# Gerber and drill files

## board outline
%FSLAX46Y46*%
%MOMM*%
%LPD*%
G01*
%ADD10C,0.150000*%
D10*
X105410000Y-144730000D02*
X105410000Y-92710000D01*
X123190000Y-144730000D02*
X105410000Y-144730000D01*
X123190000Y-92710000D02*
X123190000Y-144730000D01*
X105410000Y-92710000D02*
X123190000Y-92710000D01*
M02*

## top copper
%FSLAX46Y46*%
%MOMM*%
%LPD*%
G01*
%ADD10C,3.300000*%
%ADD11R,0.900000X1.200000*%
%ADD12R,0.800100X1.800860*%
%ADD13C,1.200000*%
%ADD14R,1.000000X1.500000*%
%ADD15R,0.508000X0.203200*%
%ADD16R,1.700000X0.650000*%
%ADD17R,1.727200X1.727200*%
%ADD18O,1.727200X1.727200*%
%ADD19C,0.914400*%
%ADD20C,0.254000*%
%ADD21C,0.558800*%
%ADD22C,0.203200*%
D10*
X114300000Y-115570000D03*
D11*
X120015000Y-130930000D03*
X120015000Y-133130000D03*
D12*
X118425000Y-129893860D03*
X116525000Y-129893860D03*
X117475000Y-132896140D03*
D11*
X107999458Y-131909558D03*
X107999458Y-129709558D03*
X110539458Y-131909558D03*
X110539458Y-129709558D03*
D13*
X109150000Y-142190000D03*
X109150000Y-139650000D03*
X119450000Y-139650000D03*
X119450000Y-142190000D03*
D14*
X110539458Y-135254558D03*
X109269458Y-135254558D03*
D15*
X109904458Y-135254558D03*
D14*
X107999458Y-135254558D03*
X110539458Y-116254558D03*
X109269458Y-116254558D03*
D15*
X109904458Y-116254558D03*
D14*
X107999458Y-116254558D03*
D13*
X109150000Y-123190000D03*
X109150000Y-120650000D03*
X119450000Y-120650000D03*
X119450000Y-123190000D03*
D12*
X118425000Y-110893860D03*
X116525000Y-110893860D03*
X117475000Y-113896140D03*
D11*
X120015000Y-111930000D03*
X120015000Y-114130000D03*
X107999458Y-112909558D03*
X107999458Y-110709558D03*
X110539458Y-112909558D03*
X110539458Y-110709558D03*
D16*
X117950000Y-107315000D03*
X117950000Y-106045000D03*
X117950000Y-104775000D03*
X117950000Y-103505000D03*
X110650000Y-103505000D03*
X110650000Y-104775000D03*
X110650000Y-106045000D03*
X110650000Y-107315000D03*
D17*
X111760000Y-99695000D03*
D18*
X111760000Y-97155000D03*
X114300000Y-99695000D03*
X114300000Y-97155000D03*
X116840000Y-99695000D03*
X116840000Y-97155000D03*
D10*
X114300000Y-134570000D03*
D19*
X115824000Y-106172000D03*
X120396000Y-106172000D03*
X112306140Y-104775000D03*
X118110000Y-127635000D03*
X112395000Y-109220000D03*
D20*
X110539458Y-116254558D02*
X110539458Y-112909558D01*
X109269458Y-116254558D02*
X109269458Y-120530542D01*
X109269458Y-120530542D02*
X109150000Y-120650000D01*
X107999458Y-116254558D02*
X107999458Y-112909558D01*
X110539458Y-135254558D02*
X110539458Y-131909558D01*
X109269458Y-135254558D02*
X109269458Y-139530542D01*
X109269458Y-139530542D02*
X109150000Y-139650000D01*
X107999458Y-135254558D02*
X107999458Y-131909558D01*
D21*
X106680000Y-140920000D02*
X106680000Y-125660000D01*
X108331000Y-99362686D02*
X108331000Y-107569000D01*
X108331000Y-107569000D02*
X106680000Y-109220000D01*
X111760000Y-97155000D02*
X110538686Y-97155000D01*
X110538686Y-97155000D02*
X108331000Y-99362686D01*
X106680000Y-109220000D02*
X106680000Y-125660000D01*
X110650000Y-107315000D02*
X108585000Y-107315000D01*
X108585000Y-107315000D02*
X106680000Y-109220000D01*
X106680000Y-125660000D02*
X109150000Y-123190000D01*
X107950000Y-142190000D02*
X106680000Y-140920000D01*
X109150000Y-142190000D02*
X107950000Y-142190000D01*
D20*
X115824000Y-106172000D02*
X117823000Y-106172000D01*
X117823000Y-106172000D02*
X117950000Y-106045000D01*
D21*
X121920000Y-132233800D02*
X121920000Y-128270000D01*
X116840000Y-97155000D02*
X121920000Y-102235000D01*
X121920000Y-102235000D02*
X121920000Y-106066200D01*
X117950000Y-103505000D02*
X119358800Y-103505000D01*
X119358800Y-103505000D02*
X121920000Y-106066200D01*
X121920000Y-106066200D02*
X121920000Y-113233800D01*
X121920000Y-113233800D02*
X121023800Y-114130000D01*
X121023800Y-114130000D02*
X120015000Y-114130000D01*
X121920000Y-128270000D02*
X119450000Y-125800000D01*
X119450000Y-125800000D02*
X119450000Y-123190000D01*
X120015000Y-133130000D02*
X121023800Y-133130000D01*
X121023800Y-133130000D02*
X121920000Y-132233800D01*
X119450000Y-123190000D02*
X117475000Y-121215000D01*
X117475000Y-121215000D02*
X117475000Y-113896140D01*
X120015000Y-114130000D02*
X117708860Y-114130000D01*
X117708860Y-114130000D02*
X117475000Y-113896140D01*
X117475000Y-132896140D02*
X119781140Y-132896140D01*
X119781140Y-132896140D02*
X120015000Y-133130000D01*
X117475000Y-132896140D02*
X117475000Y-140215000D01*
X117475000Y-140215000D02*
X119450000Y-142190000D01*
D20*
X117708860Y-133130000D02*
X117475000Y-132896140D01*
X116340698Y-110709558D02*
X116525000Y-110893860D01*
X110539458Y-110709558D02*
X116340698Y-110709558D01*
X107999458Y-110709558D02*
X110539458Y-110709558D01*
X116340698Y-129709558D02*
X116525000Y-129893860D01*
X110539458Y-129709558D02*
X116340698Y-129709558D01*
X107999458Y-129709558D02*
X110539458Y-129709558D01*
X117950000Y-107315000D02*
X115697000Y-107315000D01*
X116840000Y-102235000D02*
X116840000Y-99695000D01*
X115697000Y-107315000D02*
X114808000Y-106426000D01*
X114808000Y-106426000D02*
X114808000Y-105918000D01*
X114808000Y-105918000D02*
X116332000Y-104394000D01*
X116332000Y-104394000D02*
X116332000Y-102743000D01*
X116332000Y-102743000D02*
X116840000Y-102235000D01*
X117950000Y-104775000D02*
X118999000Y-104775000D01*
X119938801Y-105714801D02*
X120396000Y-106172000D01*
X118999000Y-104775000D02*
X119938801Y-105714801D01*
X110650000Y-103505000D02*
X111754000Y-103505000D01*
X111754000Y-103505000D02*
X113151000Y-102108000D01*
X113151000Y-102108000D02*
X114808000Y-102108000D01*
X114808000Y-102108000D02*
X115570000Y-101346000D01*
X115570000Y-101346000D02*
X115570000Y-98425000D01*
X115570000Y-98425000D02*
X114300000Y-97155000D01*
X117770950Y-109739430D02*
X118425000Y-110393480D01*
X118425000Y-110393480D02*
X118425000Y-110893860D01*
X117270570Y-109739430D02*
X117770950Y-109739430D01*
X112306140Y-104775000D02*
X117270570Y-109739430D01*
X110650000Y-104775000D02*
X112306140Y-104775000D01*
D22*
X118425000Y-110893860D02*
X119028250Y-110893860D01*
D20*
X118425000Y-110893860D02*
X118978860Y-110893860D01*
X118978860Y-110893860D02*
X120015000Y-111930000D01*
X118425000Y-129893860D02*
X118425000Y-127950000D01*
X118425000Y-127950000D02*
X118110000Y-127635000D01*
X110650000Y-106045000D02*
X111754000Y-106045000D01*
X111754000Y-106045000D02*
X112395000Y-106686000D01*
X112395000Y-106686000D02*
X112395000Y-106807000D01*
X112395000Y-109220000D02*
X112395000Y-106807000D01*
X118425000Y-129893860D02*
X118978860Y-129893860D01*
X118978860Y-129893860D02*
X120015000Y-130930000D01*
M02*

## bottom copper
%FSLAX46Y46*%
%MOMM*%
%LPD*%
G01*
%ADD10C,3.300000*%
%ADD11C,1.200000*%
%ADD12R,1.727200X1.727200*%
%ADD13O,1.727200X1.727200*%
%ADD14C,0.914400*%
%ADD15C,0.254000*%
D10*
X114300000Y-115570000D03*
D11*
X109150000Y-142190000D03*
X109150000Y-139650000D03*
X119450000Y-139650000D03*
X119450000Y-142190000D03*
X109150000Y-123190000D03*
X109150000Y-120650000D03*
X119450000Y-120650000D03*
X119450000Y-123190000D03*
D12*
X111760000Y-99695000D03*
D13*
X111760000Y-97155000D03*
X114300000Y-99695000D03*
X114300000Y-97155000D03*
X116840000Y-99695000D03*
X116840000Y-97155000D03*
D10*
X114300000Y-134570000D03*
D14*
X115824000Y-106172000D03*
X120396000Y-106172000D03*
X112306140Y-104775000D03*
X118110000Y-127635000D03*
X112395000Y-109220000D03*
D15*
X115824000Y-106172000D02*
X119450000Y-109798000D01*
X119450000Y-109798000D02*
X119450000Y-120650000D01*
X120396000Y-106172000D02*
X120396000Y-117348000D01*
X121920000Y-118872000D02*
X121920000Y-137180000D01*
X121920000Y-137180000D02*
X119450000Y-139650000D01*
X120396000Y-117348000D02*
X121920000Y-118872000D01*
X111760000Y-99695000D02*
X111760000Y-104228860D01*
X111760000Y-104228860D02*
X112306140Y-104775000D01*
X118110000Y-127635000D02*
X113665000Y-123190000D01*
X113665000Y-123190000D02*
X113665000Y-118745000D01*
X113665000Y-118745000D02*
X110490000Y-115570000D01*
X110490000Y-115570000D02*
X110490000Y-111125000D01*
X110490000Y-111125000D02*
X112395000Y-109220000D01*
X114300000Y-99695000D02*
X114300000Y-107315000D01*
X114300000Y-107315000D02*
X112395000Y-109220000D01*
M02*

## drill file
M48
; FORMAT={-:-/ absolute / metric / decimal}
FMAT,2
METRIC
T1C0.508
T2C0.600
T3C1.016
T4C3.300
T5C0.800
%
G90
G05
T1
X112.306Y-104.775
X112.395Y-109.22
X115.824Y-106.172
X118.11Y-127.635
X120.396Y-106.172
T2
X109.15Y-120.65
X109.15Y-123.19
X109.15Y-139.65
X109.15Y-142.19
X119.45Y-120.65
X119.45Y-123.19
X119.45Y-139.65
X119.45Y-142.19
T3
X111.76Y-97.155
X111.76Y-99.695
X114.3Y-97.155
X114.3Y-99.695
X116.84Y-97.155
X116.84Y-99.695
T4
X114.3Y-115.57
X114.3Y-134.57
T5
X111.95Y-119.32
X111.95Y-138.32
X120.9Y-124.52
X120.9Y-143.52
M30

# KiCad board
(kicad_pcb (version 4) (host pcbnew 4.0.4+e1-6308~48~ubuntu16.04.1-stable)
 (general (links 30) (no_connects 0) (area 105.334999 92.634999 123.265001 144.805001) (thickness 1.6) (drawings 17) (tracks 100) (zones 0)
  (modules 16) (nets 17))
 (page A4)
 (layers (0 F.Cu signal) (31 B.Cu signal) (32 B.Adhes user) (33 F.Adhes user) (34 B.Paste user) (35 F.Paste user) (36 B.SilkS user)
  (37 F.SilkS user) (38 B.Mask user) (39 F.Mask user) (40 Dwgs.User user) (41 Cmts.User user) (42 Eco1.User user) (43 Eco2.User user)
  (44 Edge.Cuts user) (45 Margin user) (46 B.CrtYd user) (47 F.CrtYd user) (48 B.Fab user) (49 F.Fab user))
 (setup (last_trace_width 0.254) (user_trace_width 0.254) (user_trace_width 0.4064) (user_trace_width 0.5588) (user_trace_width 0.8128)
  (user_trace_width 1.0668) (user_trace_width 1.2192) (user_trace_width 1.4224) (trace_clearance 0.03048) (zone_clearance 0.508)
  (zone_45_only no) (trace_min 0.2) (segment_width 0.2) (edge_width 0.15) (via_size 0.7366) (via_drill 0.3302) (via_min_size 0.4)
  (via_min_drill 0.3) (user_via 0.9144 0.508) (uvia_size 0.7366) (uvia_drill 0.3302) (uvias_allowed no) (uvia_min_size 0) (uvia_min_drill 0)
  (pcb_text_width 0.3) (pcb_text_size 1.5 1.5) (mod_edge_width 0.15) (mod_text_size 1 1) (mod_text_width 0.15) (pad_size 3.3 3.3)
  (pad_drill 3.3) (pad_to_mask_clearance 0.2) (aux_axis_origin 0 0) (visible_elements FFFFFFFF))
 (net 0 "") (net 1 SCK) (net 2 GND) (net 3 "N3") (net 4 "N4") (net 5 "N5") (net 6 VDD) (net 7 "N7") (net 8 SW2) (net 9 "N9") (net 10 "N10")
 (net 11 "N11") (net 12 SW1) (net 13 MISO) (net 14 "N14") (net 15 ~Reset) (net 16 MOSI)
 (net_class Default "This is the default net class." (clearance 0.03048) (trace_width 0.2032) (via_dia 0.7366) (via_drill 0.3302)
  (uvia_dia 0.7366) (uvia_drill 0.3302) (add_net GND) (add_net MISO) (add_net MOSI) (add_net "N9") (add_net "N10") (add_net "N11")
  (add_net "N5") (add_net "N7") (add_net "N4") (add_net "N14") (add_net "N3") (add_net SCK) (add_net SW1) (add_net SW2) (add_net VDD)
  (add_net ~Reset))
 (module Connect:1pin (layer F.Cu) (at 114.3 115.57)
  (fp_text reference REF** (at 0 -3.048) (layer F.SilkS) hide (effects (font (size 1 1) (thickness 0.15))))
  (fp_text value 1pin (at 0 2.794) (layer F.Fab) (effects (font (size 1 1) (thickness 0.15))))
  (pad 1 thru_hole circle (at 0 0) (size 3.3 3.3) (drill 3.3) (layers *.Cu *.Mask F.SilkS)))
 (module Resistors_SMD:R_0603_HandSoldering (layer F.Cu) (at 120.015 132.03 270)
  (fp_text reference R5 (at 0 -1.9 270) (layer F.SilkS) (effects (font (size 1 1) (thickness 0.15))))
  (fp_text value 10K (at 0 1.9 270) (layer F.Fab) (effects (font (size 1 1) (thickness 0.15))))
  (pad 1 smd rect (at -1.1 0 270) (size 1.2 0.9) (layers F.Cu F.Paste F.Mask) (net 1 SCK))
  (pad 2 smd rect (at 1.1 0 270) (size 1.2 0.9) (layers F.Cu F.Paste F.Mask) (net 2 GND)))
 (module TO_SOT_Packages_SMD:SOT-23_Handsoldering (layer F.Cu) (at 117.475 131.395 180)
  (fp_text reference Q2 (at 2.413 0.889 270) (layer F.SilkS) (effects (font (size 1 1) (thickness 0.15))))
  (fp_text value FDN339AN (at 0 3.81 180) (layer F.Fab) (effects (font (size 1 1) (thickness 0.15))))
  (pad 1 smd rect (at -0.95 1.50114 180) (size 0.8001 1.80086) (layers F.Cu F.Paste F.Mask) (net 1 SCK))
  (pad 2 smd rect (at 0.95 1.50114 180) (size 0.8001 1.80086) (layers F.Cu F.Paste F.Mask) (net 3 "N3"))
  (pad 3 smd rect (at 0 -1.50114 180) (size 0.8001 1.80086) (layers F.Cu F.Paste F.Mask) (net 2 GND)))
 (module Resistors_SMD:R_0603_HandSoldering (layer F.Cu) (at 107.999458 130.809558 90)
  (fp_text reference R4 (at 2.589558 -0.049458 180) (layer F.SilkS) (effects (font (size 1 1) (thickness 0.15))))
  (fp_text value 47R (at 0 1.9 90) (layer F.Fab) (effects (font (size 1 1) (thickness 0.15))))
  (pad 1 smd rect (at -1.1 0 90) (size 1.2 0.9) (layers F.Cu F.Paste F.Mask) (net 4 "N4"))
  (pad 2 smd rect (at 1.1 0 90) (size 1.2 0.9) (layers F.Cu F.Paste F.Mask) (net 3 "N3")))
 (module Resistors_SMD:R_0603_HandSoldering (layer F.Cu) (at 110.539458 130.809558 90)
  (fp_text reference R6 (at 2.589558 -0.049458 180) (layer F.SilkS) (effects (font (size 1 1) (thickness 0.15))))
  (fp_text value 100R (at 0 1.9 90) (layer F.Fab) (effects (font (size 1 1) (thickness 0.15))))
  (pad 1 smd rect (at -1.1 0 90) (size 1.2 0.9) (layers F.Cu F.Paste F.Mask) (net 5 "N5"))
  (pad 2 smd rect (at 1.1 0 90) (size 1.2 0.9) (layers F.Cu F.Paste F.Mask) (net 3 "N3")))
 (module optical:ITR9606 (layer F.Cu) (at 114.3 140.92)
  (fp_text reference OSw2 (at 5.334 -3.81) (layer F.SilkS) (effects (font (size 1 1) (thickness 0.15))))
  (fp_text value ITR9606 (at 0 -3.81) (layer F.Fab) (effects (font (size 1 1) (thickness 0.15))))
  (pad 1 thru_hole circle (at -5.15 1.27) (size 1.2 1.2) (drill 0.6) (layers *.Cu *.Mask) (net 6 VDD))
  (pad 2 thru_hole circle (at -5.15 -1.27) (size 1.2 1.2) (drill 0.6) (layers *.Cu *.Mask) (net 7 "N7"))
  (pad 3 thru_hole circle (at 5.15 -1.27) (size 1.2 1.2) (drill 0.6) (layers *.Cu *.Mask) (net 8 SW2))
  (pad 4 thru_hole circle (at 5.15 1.27) (size 1.2 1.2) (drill 0.6) (layers *.Cu *.Mask) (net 2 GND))
  (pad "" np_thru_hole circle (at -2.35 -2.6) (size 0.8 0.8) (drill 0.8) (layers *.Cu *.Mask))
  (pad "" np_thru_hole circle (at 6.6 2.6) (size 0.8 0.8) (drill 0.8) (layers *.Cu *.Mask)))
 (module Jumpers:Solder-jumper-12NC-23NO (layer F.Cu) (at 109.904458 135.254558 180)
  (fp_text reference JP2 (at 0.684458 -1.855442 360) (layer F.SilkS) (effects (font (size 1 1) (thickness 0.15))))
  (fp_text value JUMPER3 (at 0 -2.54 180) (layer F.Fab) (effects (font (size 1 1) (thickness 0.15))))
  (pad 1 smd rect (at -0.635 0 180) (size 1 1.5) (layers F.Cu F.Paste F.Mask) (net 5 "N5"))
  (pad 2 smd rect (at 0.635 0 180) (size 1 1.5) (layers F.Cu F.Paste F.Mask) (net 7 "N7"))
  (pad "" smd rect (at 0 0 270) (size 0.2032 0.508) (layers F.Cu F.Paste F.Mask))
  (pad 3 smd rect (at 1.905 0 180) (size 1 1.5) (layers F.Cu F.Paste F.Mask) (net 4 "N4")))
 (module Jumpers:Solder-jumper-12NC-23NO (layer F.Cu) (at 109.904458 116.254558 180)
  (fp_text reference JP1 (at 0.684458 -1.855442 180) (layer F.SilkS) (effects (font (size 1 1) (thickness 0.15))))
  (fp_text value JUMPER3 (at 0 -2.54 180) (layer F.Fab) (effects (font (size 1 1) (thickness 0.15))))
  (pad 1 smd rect (at -0.635 0 180) (size 1 1.5) (layers F.Cu F.Paste F.Mask) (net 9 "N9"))
  (pad 2 smd rect (at 0.635 0 180) (size 1 1.5) (layers F.Cu F.Paste F.Mask) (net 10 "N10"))
  (pad "" smd rect (at 0 0 270) (size 0.2032 0.508) (layers F.Cu F.Paste F.Mask))
  (pad 3 smd rect (at 1.905 0 180) (size 1 1.5) (layers F.Cu F.Paste F.Mask) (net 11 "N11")))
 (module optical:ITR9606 (layer F.Cu) (at 114.3 121.92)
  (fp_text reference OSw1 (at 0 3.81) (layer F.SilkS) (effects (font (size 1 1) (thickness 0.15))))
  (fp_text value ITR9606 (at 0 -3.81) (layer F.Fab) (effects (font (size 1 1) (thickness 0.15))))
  (pad 1 thru_hole circle (at -5.15 1.27) (size 1.2 1.2) (drill 0.6) (layers *.Cu *.Mask) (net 6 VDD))
  (pad 2 thru_hole circle (at -5.15 -1.27) (size 1.2 1.2) (drill 0.6) (layers *.Cu *.Mask) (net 10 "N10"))
  (pad 3 thru_hole circle (at 5.15 -1.27) (size 1.2 1.2) (drill 0.6) (layers *.Cu *.Mask) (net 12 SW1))
  (pad 4 thru_hole circle (at 5.15 1.27) (size 1.2 1.2) (drill 0.6) (layers *.Cu *.Mask) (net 2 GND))
  (pad "" np_thru_hole circle (at -2.35 -2.6) (size 0.8 0.8) (drill 0.8) (layers *.Cu *.Mask))
  (pad "" np_thru_hole circle (at 6.6 2.6) (size 0.8 0.8) (drill 0.8) (layers *.Cu *.Mask)))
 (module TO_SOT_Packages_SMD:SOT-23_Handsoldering (layer F.Cu) (at 117.475 112.395 180)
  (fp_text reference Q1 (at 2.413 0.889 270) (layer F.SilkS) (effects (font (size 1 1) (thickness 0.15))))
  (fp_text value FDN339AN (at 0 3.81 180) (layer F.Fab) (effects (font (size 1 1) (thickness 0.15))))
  (pad 1 smd rect (at -0.95 1.50114 180) (size 0.8001 1.80086) (layers F.Cu F.Paste F.Mask) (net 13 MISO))
  (pad 2 smd rect (at 0.95 1.50114 180) (size 0.8001 1.80086) (layers F.Cu F.Paste F.Mask) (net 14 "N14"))
  (pad 3 smd rect (at 0 -1.50114 180) (size 0.8001 1.80086) (layers F.Cu F.Paste F.Mask) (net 2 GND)))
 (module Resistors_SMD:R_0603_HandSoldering (layer F.Cu) (at 120.015 113.03 270)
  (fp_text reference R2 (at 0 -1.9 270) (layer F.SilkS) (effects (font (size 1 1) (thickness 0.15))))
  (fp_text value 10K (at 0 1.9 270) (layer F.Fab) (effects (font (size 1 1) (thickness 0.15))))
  (pad 1 smd rect (at -1.1 0 270) (size 1.2 0.9) (layers F.Cu F.Paste F.Mask) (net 13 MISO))
  (pad 2 smd rect (at 1.1 0 270) (size 1.2 0.9) (layers F.Cu F.Paste F.Mask) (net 2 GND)))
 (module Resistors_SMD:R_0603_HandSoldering (layer F.Cu) (at 107.999458 111.809558 90)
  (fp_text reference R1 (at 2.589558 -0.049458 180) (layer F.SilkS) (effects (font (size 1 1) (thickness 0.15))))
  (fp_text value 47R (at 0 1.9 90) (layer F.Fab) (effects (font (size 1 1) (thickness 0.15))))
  (pad 1 smd rect (at -1.1 0 90) (size 1.2 0.9) (layers F.Cu F.Paste F.Mask) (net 11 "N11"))
  (pad 2 smd rect (at 1.1 0 90) (size 1.2 0.9) (layers F.Cu F.Paste F.Mask) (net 14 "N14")))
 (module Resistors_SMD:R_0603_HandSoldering (layer F.Cu) (at 110.539458 111.809558 90)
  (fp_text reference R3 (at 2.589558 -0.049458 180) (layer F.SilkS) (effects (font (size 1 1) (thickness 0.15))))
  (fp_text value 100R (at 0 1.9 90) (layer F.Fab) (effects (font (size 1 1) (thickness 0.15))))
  (pad 1 smd rect (at -1.1 0 90) (size 1.2 0.9) (layers F.Cu F.Paste F.Mask) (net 9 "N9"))
  (pad 2 smd rect (at 1.1 0 90) (size 1.2 0.9) (layers F.Cu F.Paste F.Mask) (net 14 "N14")))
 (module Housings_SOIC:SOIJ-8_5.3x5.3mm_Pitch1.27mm (layer F.Cu) (at 114.3 105.41 180)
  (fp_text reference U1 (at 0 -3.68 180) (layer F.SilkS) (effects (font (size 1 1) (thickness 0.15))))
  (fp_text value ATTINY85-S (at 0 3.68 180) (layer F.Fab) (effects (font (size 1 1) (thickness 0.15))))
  (pad 1 smd rect (at -3.65 -1.905 180) (size 1.7 0.65) (layers F.Cu F.Paste F.Mask) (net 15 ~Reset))
  (pad 2 smd rect (at -3.65 -0.635 180) (size 1.7 0.65) (layers F.Cu F.Paste F.Mask) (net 12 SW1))
  (pad 3 smd rect (at -3.65 0.635 180) (size 1.7 0.65) (layers F.Cu F.Paste F.Mask) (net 8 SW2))
  (pad 4 smd rect (at -3.65 1.905 180) (size 1.7 0.65) (layers F.Cu F.Paste F.Mask) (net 2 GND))
  (pad 5 smd rect (at 3.65 1.905 180) (size 1.7 0.65) (layers F.Cu F.Paste F.Mask) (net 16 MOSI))
  (pad 6 smd rect (at 3.65 0.635 180) (size 1.7 0.65) (layers F.Cu F.Paste F.Mask) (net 13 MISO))
  (pad 7 smd rect (at 3.65 -0.635 180) (size 1.7 0.65) (layers F.Cu F.Paste F.Mask) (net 1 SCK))
  (pad 8 smd rect (at 3.65 -1.905 180) (size 1.7 0.65) (layers F.Cu F.Paste F.Mask) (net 6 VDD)))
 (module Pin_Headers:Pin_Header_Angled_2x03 (layer F.Cu) (at 111.76 99.695 90)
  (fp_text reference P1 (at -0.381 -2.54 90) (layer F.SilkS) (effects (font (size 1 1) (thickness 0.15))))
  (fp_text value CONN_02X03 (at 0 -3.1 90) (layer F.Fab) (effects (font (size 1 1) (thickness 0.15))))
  (pad 1 thru_hole rect (at 0 0 90) (size 1.7272 1.7272) (drill 1.016) (layers *.Cu *.Mask F.SilkS) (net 13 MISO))
  (pad 2 thru_hole oval (at 2.54 0 90) (size 1.7272 1.7272) (drill 1.016) (layers *.Cu *.Mask F.SilkS) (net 6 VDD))
  (pad 3 thru_hole oval (at 0 2.54 90) (size 1.7272 1.7272) (drill 1.016) (layers *.Cu *.Mask F.SilkS) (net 1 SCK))
  (pad 4 thru_hole oval (at 2.54 2.54 90) (size 1.7272 1.7272) (drill 1.016) (layers *.Cu *.Mask F.SilkS) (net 16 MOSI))
  (pad 5 thru_hole oval (at 0 5.08 90) (size 1.7272 1.7272) (drill 1.016) (layers *.Cu *.Mask F.SilkS) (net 15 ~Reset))
  (pad 6 thru_hole oval (at 2.54 5.08 90) (size 1.7272 1.7272) (drill 1.016) (layers *.Cu *.Mask F.SilkS) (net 2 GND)))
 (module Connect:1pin (layer F.Cu) (at 114.3 134.57)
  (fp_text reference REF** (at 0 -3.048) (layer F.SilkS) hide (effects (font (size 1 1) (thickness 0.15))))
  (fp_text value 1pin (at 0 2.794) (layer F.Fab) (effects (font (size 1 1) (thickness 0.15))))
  (pad 1 thru_hole circle (at 0 0) (size 3.3 3.3) (drill 3.3) (layers *.Cu *.Mask F.SilkS)))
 (gr_line (start 105.41 144.73) (end 105.41 92.71) (layer Edge.Cuts) (width 0.15))
 (gr_line (start 123.19 144.73) (end 105.41 144.73) (layer Edge.Cuts) (width 0.15))
 (gr_line (start 123.19 92.71) (end 123.19 144.73) (layer Edge.Cuts) (width 0.15))
 (gr_line (start 105.41 92.71) (end 123.19 92.71) (layer Edge.Cuts) (width 0.15))
 (segment (start 110.539458 116.254558) (end 110.539458 112.909558) (width 0.254) (layer F.Cu) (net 9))
 (segment (start 109.269458 116.254558) (end 109.269458 120.530542) (width 0.254) (layer F.Cu) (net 10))
 (segment (start 109.269458 120.530542) (end 109.15 120.65) (width 0.254) (layer F.Cu) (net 10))
 (segment (start 107.999458 116.254558) (end 107.999458 112.909558) (width 0.254) (layer F.Cu) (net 11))
 (segment (start 110.539458 135.254558) (end 110.539458 131.909558) (width 0.254) (layer F.Cu) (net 5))
 (segment (start 109.269458 135.254558) (end 109.269458 139.530542) (width 0.254) (layer F.Cu) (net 7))
 (segment (start 109.269458 139.530542) (end 109.15 139.65) (width 0.254) (layer F.Cu) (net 7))
 (segment (start 107.999458 135.254558) (end 107.999458 131.909558) (width 0.254) (layer F.Cu) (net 4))
 (segment (start 106.68 140.92) (end 106.68 125.66) (width 0.5588) (layer F.Cu) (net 6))
 (segment (start 108.331 99.362686) (end 108.331 107.569) (width 0.5588) (layer F.Cu) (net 6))
 (segment (start 108.331 107.569) (end 106.68 109.22) (width 0.5588) (layer F.Cu) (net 6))
 (segment (start 111.76 97.155) (end 110.538686 97.155) (width 0.5588) (layer F.Cu) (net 6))
 (segment (start 110.538686 97.155) (end 108.331 99.362686) (width 0.5588) (layer F.Cu) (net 6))
 (segment (start 106.68 109.22) (end 106.68 125.66) (width 0.5588) (layer F.Cu) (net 6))
 (segment (start 110.65 107.315) (end 108.585 107.315) (width 0.5588) (layer F.Cu) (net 6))
 (segment (start 108.585 107.315) (end 106.68 109.22) (width 0.5588) (layer F.Cu) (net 6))
 (segment (start 106.68 125.66) (end 109.15 123.19) (width 0.5588) (layer F.Cu) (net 6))
 (segment (start 107.95 142.19) (end 106.68 140.92) (width 0.5588) (layer F.Cu) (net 6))
 (segment (start 109.15 142.19) (end 107.95 142.19) (width 0.5588) (layer F.Cu) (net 6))
 (segment (start 115.824 106.172) (end 117.823 106.172) (width 0.254) (layer F.Cu) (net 12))
 (segment (start 117.823 106.172) (end 117.95 106.045) (width 0.254) (layer F.Cu) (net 12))
 (segment (start 115.824 106.172) (end 119.45 109.798) (width 0.254) (layer B.Cu) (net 12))
 (segment (start 119.45 109.798) (end 119.45 120.65) (width 0.254) (layer B.Cu) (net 12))
 (via (at 115.824 106.172) (size 0.9144) (drill 0.508) (layers F.Cu B.Cu) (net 12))
 (segment (start 121.92 132.2338) (end 121.92 128.27) (width 0.5588) (layer F.Cu) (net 2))
 (segment (start 116.84 97.155) (end 121.92 102.235) (width 0.5588) (layer F.Cu) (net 2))
 (segment (start 121.92 102.235) (end 121.92 106.0662) (width 0.5588) (layer F.Cu) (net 2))
 (segment (start 117.95 103.505) (end 119.3588 103.505) (width 0.5588) (layer F.Cu) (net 2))
 (segment (start 119.3588 103.505) (end 121.92 106.0662) (width 0.5588) (layer F.Cu) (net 2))
 (segment (start 121.92 106.0662) (end 121.92 113.2338) (width 0.5588) (layer F.Cu) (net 2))
 (segment (start 121.92 113.2338) (end 121.0238 114.13) (width 0.5588) (layer F.Cu) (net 2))
 (segment (start 121.0238 114.13) (end 120.015 114.13) (width 0.5588) (layer F.Cu) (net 2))
 (segment (start 121.92 128.27) (end 119.45 125.8) (width 0.5588) (layer F.Cu) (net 2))
 (segment (start 119.45 125.8) (end 119.45 123.19) (width 0.5588) (layer F.Cu) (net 2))
 (segment (start 120.015 133.13) (end 121.0238 133.13) (width 0.5588) (layer F.Cu) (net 2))
 (segment (start 121.0238 133.13) (end 121.92 132.2338) (width 0.5588) (layer F.Cu) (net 2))
 (segment (start 119.45 123.19) (end 117.475 121.215) (width 0.5588) (layer F.Cu) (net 2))
 (segment (start 117.475 121.215) (end 117.475 113.89614) (width 0.5588) (layer F.Cu) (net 2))
 (segment (start 120.015 114.13) (end 117.70886 114.13) (width 0.5588) (layer F.Cu) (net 2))
 (segment (start 117.70886 114.13) (end 117.475 113.89614) (width 0.5588) (layer F.Cu) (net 2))
 (segment (start 117.475 132.89614) (end 119.78114 132.89614) (width 0.5588) (layer F.Cu) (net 2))
 (segment (start 119.78114 132.89614) (end 120.015 133.13) (width 0.5588) (layer F.Cu) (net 2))
 (segment (start 117.475 132.89614) (end 117.475 140.215) (width 0.5588) (layer F.Cu) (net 2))
 (segment (start 117.475 140.215) (end 119.45 142.19) (width 0.5588) (layer F.Cu) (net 2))
 (segment (start 117.70886 133.13) (end 117.475 132.89614) (width 0.254) (layer F.Cu) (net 2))
 (segment (start 116.340698 110.709558) (end 116.525 110.89386) (width 0.254) (layer F.Cu) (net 14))
 (segment (start 110.539458 110.709558) (end 116.340698 110.709558) (width 0.254) (layer F.Cu) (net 14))
 (segment (start 107.999458 110.709558) (end 110.539458 110.709558) (width 0.254) (layer F.Cu) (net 14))
 (segment (start 116.340698 129.709558) (end 116.525 129.89386) (width 0.254) (layer F.Cu) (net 3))
 (segment (start 110.539458 129.709558) (end 116.340698 129.709558) (width 0.254) (layer F.Cu) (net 3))
 (segment (start 107.999458 129.709558) (end 110.539458 129.709558) (width 0.254) (layer F.Cu) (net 3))
 (segment (start 117.95 107.315) (end 115.697 107.315) (width 0.254) (layer F.Cu) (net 15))
 (segment (start 116.84 102.235) (end 116.84 99.695) (width 0.254) (layer F.Cu) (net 15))
 (segment (start 115.697 107.315) (end 114.808 106.426) (width 0.254) (layer F.Cu) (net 15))
 (segment (start 114.808 106.426) (end 114.808 105.918) (width 0.254) (layer F.Cu) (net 15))
 (segment (start 114.808 105.918) (end 116.332 104.394) (width 0.254) (layer F.Cu) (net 15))
 (segment (start 116.332 104.394) (end 116.332 102.743) (width 0.254) (layer F.Cu) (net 15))
 (segment (start 116.332 102.743) (end 116.84 102.235) (width 0.254) (layer F.Cu) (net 15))
 (segment (start 120.396 106.172) (end 120.396 117.348) (width 0.254) (layer B.Cu) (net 8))
 (segment (start 121.92 118.872) (end 121.92 137.18) (width 0.254) (layer B.Cu) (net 8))
 (segment (start 121.92 137.18) (end 119.45 139.65) (width 0.254) (layer B.Cu) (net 8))
 (segment (start 120.396 117.348) (end 121.92 118.872) (width 0.254) (layer B.Cu) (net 8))
 (segment (start 117.95 104.775) (end 118.999 104.775) (width 0.254) (layer F.Cu) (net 8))
 (segment (start 119.938801 105.714801) (end 120.396 106.172) (width 0.254) (layer F.Cu) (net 8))
 (segment (start 118.999 104.775) (end 119.938801 105.714801) (width 0.254) (layer F.Cu) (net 8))
 (via (at 120.396 106.172) (size 0.9144) (drill 0.508) (layers F.Cu B.Cu) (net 8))
 (segment (start 110.65 103.505) (end 111.754 103.505) (width 0.254) (layer F.Cu) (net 16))
 (segment (start 111.754 103.505) (end 113.151 102.108) (width 0.254) (layer F.Cu) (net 16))
 (segment (start 113.151 102.108) (end 114.808 102.108) (width 0.254) (layer F.Cu) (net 16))
 (segment (start 114.808 102.108) (end 115.57 101.346) (width 0.254) (layer F.Cu) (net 16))
 (segment (start 115.57 101.346) (end 115.57 98.425) (width 0.254) (layer F.Cu) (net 16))
 (segment (start 115.57 98.425) (end 114.3 97.155) (width 0.254) (layer F.Cu) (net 16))
 (segment (start 111.76 99.695) (end 111.76 104.22886) (width 0.254) (layer B.Cu) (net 13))
 (via (at 112.30614 104.775) (size 0.9144) (drill 0.508) (layers F.Cu B.Cu) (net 13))
 (segment (start 111.76 104.22886) (end 112.30614 104.775) (width 0.254) (layer B.Cu) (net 13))
 (segment (start 117.77095 109.73943) (end 118.425 110.39348) (width 0.254) (layer F.Cu) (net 13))
 (segment (start 118.425 110.39348) (end 118.425 110.89386) (width 0.254) (layer F.Cu) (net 13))
 (segment (start 117.27057 109.73943) (end 117.77095 109.73943) (width 0.254) (layer F.Cu) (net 13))
 (segment (start 112.30614 104.775) (end 117.27057 109.73943) (width 0.254) (layer F.Cu) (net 13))
 (segment (start 110.65 104.775) (end 112.30614 104.775) (width 0.254) (layer F.Cu) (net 13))
 (segment (start 118.425 110.89386) (end 119.02825 110.89386) (width 0.2032) (layer F.Cu) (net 13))
 (segment (start 118.425 110.89386) (end 118.97886 110.89386) (width 0.254) (layer F.Cu) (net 13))
 (segment (start 118.97886 110.89386) (end 120.015 111.93) (width 0.254) (layer F.Cu) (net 13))
 (segment (start 118.425 129.89386) (end 118.425 127.95) (width 0.254) (layer F.Cu) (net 1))
 (segment (start 118.425 127.95) (end 118.11 127.635) (width 0.254) (layer F.Cu) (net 1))
 (segment (start 118.11 127.635) (end 113.665 123.19) (width 0.254) (layer B.Cu) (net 1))
 (segment (start 113.665 123.19) (end 113.665 118.745) (width 0.254) (layer B.Cu) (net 1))
 (segment (start 113.665 118.745) (end 110.49 115.57) (width 0.254) (layer B.Cu) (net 1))
 (segment (start 110.49 115.57) (end 110.49 111.125) (width 0.254) (layer B.Cu) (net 1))
 (segment (start 110.49 111.125) (end 112.395 109.22) (width 0.254) (layer B.Cu) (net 1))
 (segment (start 114.3 99.695) (end 114.3 107.315) (width 0.254) (layer B.Cu) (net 1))
 (segment (start 114.3 107.315) (end 112.395 109.22) (width 0.254) (layer B.Cu) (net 1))
 (segment (start 110.65 106.045) (end 111.754 106.045) (width 0.254) (layer F.Cu) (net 1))
 (segment (start 111.754 106.045) (end 112.395 106.686) (width 0.254) (layer F.Cu) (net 1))
 (segment (start 112.395 106.686) (end 112.395 106.807) (width 0.254) (layer F.Cu) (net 1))
 (segment (start 112.395 109.22) (end 112.395 106.807) (width 0.254) (layer F.Cu) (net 1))
 (via (at 118.11 127.635) (size 0.9144) (drill 0.508) (layers F.Cu B.Cu) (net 1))
 (via (at 112.395 109.22) (size 0.9144) (drill 0.508) (layers F.Cu B.Cu) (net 1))
 (segment (start 118.425 129.89386) (end 118.97886 129.89386) (width 0.254) (layer F.Cu) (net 1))
 (segment (start 118.97886 129.89386) (end 120.015 130.93) (width 0.254) (layer F.Cu) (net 1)))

